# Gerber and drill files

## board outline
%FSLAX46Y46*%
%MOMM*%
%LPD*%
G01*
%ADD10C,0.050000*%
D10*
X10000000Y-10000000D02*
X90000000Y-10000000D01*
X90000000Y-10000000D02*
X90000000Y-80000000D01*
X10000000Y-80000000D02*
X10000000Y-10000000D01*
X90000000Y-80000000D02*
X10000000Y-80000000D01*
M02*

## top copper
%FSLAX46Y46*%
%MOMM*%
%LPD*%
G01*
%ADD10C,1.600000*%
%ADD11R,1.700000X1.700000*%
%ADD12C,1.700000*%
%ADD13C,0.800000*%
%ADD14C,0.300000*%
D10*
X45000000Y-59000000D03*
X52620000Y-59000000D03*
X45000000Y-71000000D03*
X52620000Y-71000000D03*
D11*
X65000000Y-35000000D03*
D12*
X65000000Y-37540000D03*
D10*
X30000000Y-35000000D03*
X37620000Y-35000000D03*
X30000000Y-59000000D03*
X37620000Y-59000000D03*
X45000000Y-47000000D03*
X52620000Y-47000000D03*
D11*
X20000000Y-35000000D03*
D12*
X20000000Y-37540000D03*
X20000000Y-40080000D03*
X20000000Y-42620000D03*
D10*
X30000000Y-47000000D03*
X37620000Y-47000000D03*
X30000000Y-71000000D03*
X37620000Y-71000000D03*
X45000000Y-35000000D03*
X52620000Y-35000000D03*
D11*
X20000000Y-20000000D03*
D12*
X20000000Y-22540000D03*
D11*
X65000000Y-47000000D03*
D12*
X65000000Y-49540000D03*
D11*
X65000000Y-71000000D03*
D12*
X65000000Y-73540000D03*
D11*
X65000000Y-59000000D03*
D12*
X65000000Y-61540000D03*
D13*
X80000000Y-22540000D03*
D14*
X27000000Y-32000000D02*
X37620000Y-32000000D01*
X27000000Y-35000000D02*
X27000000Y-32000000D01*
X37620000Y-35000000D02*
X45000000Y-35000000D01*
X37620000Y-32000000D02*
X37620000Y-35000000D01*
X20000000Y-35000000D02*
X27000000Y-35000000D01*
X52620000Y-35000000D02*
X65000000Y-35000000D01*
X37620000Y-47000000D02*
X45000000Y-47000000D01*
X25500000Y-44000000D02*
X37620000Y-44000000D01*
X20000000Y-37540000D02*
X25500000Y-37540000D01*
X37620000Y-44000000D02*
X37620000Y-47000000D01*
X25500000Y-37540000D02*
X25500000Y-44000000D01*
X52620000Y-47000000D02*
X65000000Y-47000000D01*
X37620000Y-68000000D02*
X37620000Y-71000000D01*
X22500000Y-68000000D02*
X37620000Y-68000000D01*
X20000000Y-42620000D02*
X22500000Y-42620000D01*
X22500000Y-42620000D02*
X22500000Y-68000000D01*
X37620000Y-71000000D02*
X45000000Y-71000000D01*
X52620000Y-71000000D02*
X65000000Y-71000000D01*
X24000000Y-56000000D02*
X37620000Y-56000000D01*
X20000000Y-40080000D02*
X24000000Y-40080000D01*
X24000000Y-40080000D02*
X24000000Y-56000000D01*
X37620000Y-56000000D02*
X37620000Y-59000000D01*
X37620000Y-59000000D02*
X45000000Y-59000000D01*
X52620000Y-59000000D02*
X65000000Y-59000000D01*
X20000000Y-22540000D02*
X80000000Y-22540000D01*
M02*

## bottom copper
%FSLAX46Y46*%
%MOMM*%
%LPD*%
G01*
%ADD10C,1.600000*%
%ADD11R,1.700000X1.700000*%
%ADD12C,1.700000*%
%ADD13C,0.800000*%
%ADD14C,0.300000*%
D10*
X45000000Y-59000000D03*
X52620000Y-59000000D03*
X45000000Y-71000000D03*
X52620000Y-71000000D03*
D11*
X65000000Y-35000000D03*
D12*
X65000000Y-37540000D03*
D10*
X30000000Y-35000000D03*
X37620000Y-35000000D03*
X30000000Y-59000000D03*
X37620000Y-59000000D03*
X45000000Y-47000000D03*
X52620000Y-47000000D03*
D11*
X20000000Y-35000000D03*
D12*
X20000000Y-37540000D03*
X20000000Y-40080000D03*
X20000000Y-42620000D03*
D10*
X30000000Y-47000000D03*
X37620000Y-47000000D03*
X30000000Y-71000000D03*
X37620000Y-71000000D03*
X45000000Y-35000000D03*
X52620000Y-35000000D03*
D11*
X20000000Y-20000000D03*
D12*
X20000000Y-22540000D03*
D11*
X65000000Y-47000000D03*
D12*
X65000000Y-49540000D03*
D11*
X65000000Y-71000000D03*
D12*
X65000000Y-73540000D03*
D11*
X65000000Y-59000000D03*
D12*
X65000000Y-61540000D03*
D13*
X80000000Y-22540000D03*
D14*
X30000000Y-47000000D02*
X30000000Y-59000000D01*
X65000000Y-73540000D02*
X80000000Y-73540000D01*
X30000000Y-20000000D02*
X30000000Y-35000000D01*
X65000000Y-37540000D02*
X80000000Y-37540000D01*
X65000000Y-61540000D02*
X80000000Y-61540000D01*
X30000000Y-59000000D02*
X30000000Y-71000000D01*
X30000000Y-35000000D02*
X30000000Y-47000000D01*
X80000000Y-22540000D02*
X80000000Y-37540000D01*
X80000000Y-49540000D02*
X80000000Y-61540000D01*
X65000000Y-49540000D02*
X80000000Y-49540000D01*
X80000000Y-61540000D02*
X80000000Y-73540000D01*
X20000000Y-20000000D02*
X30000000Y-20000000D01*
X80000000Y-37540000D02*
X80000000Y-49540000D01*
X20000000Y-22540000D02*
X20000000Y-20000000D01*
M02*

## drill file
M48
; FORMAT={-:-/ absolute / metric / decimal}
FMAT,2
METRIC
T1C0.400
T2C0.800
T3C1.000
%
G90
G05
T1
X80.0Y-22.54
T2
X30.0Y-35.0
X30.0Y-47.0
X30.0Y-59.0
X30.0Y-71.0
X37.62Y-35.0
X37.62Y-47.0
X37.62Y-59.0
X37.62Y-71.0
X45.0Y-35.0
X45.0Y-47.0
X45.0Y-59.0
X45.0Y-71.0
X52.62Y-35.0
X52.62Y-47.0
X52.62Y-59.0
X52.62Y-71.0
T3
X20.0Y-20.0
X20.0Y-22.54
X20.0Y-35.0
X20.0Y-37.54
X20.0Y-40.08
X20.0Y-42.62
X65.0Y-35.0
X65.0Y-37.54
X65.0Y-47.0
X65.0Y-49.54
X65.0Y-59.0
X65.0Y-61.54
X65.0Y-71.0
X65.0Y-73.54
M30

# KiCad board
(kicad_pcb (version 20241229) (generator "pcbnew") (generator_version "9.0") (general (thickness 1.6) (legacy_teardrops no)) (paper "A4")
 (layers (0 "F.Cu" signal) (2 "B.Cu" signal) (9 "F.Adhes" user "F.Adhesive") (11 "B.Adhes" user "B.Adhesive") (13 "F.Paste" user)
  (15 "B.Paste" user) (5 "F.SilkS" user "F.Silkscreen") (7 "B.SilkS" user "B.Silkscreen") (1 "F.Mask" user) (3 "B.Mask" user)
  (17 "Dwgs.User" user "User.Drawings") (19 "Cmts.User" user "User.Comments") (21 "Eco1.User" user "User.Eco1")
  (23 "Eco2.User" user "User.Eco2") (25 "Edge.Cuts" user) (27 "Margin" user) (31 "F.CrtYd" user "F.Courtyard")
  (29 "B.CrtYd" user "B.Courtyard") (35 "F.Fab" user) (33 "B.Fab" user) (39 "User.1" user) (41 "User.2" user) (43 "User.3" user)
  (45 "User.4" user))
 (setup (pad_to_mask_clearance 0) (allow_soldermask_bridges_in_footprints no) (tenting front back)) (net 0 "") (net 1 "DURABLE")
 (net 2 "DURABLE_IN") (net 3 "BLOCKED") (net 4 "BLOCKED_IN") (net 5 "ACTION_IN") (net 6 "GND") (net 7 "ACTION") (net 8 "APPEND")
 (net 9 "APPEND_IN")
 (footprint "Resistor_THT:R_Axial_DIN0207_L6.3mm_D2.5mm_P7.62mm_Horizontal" (layer "F.Cu") (at 45 59)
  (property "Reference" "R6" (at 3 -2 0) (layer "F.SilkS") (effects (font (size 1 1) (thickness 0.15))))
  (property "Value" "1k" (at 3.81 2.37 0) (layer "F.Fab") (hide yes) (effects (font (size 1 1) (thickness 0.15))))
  (pad "1" thru_hole circle (at 0 0) (size 1.6 1.6) (drill 0.8) (layers "*.Cu" "*.Mask") (remove_unused_layers no) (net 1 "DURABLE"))
  (pad "2" thru_hole circle (at 7.62 0) (size 1.6 1.6) (drill 0.8) (layers "*.Cu" "*.Mask") (remove_unused_layers no) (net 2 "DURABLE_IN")))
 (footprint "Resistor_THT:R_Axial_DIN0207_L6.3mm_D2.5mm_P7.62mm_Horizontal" (layer "F.Cu") (at 45 71)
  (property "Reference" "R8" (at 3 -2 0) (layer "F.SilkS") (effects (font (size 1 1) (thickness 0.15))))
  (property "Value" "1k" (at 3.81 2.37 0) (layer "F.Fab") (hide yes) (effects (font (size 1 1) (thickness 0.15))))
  (pad "1" thru_hole circle (at 0 0) (size 1.6 1.6) (drill 0.8) (layers "*.Cu" "*.Mask") (remove_unused_layers no) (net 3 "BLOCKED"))
  (pad "2" thru_hole circle (at 7.62 0) (size 1.6 1.6) (drill 0.8) (layers "*.Cu" "*.Mask") (remove_unused_layers no) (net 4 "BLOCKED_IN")))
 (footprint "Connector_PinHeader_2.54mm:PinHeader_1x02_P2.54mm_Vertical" (layer "F.Cu") (at 65 35)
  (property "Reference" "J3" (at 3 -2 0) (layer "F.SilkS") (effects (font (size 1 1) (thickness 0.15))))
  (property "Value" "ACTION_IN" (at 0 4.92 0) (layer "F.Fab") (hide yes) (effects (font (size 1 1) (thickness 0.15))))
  (pad "1" thru_hole rect (at 0 0) (size 1.7 1.7) (drill 1) (layers "*.Cu" "*.Mask") (remove_unused_layers no) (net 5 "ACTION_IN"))
  (pad "2" thru_hole circle (at 0 2.54) (size 1.7 1.7) (drill 1) (layers "*.Cu" "*.Mask") (remove_unused_layers no) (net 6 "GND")))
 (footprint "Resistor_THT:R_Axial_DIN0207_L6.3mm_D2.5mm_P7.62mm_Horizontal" (layer "F.Cu") (at 30 35)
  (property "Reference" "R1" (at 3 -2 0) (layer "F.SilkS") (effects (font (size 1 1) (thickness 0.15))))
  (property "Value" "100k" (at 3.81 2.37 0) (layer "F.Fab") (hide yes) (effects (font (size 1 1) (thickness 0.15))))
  (pad "1" thru_hole circle (at 0 0) (size 1.6 1.6) (drill 0.8) (layers "*.Cu" "*.Mask") (remove_unused_layers no) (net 6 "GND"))
  (pad "2" thru_hole circle (at 7.62 0) (size 1.6 1.6) (drill 0.8) (layers "*.Cu" "*.Mask") (remove_unused_layers no) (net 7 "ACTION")))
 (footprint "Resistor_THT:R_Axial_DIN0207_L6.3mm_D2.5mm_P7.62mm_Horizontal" (layer "F.Cu") (at 30 59)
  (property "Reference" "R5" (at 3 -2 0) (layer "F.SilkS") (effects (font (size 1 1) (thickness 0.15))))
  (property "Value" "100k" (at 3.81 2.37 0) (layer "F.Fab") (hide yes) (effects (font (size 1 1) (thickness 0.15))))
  (pad "1" thru_hole circle (at 0 0) (size 1.6 1.6) (drill 0.8) (layers "*.Cu" "*.Mask") (remove_unused_layers no) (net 6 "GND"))
  (pad "2" thru_hole circle (at 7.62 0) (size 1.6 1.6) (drill 0.8) (layers "*.Cu" "*.Mask") (remove_unused_layers no) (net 1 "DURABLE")))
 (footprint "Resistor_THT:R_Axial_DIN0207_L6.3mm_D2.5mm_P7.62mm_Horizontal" (layer "F.Cu") (at 45 47)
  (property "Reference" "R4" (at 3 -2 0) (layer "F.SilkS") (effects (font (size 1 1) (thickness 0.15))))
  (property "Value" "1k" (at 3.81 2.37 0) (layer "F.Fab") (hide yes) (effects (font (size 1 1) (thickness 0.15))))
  (pad "1" thru_hole circle (at 0 0) (size 1.6 1.6) (drill 0.8) (layers "*.Cu" "*.Mask") (remove_unused_layers no) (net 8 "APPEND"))
  (pad "2" thru_hole circle (at 7.62 0) (size 1.6 1.6) (drill 0.8) (layers "*.Cu" "*.Mask") (remove_unused_layers no) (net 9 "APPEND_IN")))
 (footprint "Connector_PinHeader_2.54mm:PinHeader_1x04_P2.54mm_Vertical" (layer "F.Cu") (at 20 35)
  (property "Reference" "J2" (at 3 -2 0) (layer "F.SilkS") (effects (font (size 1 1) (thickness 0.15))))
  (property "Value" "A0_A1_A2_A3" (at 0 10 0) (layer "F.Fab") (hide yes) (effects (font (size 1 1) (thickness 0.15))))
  (pad "1" thru_hole rect (at 0 0) (size 1.7 1.7) (drill 1) (layers "*.Cu" "*.Mask") (remove_unused_layers no) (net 7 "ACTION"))
  (pad "2" thru_hole circle (at 0 2.54) (size 1.7 1.7) (drill 1) (layers "*.Cu" "*.Mask") (remove_unused_layers no) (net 8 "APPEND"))
  (pad "3" thru_hole circle (at 0 5.08) (size 1.7 1.7) (drill 1) (layers "*.Cu" "*.Mask") (remove_unused_layers no) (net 1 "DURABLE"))
  (pad "4" thru_hole circle (at 0 7.62) (size 1.7 1.7) (drill 1) (layers "*.Cu" "*.Mask") (remove_unused_layers no) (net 3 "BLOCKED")))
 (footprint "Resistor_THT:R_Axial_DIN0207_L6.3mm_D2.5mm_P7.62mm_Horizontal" (layer "F.Cu") (at 30 47)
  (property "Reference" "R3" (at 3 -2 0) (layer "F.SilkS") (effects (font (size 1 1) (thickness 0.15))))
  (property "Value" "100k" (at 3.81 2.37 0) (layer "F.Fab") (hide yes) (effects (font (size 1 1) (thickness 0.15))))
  (pad "1" thru_hole circle (at 0 0) (size 1.6 1.6) (drill 0.8) (layers "*.Cu" "*.Mask") (remove_unused_layers no) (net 6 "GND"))
  (pad "2" thru_hole circle (at 7.62 0) (size 1.6 1.6) (drill 0.8) (layers "*.Cu" "*.Mask") (remove_unused_layers no) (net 8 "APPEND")))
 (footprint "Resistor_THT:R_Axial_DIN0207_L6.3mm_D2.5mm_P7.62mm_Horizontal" (layer "F.Cu") (at 30 71)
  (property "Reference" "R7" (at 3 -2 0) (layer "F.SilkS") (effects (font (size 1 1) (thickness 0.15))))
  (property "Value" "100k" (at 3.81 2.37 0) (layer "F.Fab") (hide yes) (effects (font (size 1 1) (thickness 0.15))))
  (pad "1" thru_hole circle (at 0 0) (size 1.6 1.6) (drill 0.8) (layers "*.Cu" "*.Mask") (remove_unused_layers no) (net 6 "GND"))
  (pad "2" thru_hole circle (at 7.62 0) (size 1.6 1.6) (drill 0.8) (layers "*.Cu" "*.Mask") (remove_unused_layers no) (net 3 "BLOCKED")))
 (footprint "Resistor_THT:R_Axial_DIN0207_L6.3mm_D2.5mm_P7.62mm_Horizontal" (layer "F.Cu") (at 45 35)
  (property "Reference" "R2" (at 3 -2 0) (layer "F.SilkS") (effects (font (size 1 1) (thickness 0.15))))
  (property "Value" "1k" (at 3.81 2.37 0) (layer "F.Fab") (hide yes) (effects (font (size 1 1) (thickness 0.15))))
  (pad "1" thru_hole circle (at 0 0) (size 1.6 1.6) (drill 0.8) (layers "*.Cu" "*.Mask") (remove_unused_layers no) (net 7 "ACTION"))
  (pad "2" thru_hole circle (at 7.62 0) (size 1.6 1.6) (drill 0.8) (layers "*.Cu" "*.Mask") (remove_unused_layers no) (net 5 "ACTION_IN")))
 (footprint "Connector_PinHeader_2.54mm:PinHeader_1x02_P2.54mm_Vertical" (layer "F.Cu") (at 20 20)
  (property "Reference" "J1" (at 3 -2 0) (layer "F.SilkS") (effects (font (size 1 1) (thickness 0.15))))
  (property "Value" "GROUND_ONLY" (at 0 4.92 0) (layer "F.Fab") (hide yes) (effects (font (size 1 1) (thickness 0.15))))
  (pad "1" thru_hole rect (at 0 0) (size 1.7 1.7) (drill 1) (layers "*.Cu" "*.Mask") (remove_unused_layers no) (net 6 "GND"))
  (pad "2" thru_hole circle (at 0 2.54) (size 1.7 1.7) (drill 1) (layers "*.Cu" "*.Mask") (remove_unused_layers no) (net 6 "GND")))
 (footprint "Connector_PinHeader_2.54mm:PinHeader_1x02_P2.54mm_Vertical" (layer "F.Cu") (at 65 47)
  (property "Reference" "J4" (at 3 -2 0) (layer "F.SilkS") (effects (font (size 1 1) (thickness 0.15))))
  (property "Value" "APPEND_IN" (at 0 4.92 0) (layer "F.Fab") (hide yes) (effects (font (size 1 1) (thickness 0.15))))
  (pad "1" thru_hole rect (at 0 0) (size 1.7 1.7) (drill 1) (layers "*.Cu" "*.Mask") (remove_unused_layers no) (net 9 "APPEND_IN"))
  (pad "2" thru_hole circle (at 0 2.54) (size 1.7 1.7) (drill 1) (layers "*.Cu" "*.Mask") (remove_unused_layers no) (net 6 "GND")))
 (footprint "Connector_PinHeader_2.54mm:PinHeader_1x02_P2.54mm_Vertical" (layer "F.Cu") (at 65 71)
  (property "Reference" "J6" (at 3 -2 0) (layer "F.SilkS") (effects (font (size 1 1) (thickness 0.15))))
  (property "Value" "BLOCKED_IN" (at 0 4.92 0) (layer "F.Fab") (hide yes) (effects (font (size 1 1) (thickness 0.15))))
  (pad "1" thru_hole rect (at 0 0) (size 1.7 1.7) (drill 1) (layers "*.Cu" "*.Mask") (remove_unused_layers no) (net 4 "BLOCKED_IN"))
  (pad "2" thru_hole circle (at 0 2.54) (size 1.7 1.7) (drill 1) (layers "*.Cu" "*.Mask") (remove_unused_layers no) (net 6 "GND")))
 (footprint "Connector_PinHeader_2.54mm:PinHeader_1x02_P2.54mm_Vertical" (layer "F.Cu") (at 65 59)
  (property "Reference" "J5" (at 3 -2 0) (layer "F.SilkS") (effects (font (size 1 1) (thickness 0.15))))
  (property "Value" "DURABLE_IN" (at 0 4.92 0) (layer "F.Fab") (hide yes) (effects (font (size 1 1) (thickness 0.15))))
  (pad "1" thru_hole rect (at 0 0) (size 1.7 1.7) (drill 1) (layers "*.Cu" "*.Mask") (remove_unused_layers no) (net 2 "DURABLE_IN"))
  (pad "2" thru_hole circle (at 0 2.54) (size 1.7 1.7) (drill 1) (layers "*.Cu" "*.Mask") (remove_unused_layers no) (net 6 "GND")))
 (gr_line (start 10 10) (end 90 10) (stroke (width 0.05) (type default)) (layer "Edge.Cuts"))
 (gr_line (start 90 10) (end 90 80) (stroke (width 0.05) (type default)) (layer "Edge.Cuts"))
 (gr_line (start 10 80) (end 10 10) (stroke (width 0.05) (type default)) (layer "Edge.Cuts"))
 (gr_line (start 90 80) (end 10 80) (stroke (width 0.05) (type default)) (layer "Edge.Cuts"))
 (segment (start 27 32) (end 37.62 32) (width 0.3) (layer "F.Cu") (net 7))
 (segment (start 27 35) (end 27 32) (width 0.3) (layer "F.Cu") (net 7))
 (segment (start 37.62 35) (end 45 35) (width 0.3) (layer "F.Cu") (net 7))
 (segment (start 37.62 32) (end 37.62 35) (width 0.3) (layer "F.Cu") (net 7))
 (segment (start 20 35) (end 27 35) (width 0.3) (layer "F.Cu") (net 7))
 (segment (start 52.62 35) (end 65 35) (width 0.3) (layer "F.Cu") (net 5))
 (segment (start 37.62 47) (end 45 47) (width 0.3) (layer "F.Cu") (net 8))
 (segment (start 25.5 44) (end 37.62 44) (width 0.3) (layer "F.Cu") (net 8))
 (segment (start 20 37.54) (end 25.5 37.54) (width 0.3) (layer "F.Cu") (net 8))
 (segment (start 37.62 44) (end 37.62 47) (width 0.3) (layer "F.Cu") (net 8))
 (segment (start 25.5 37.54) (end 25.5 44) (width 0.3) (layer "F.Cu") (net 8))
 (segment (start 52.62 47) (end 65 47) (width 0.3) (layer "F.Cu") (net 9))
 (segment (start 37.62 68) (end 37.62 71) (width 0.3) (layer "F.Cu") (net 3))
 (segment (start 22.5 68) (end 37.62 68) (width 0.3) (layer "F.Cu") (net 3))
 (segment (start 20 42.62) (end 22.5 42.62) (width 0.3) (layer "F.Cu") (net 3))
 (segment (start 22.5 42.62) (end 22.5 68) (width 0.3) (layer "F.Cu") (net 3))
 (segment (start 37.62 71) (end 45 71) (width 0.3) (layer "F.Cu") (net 3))
 (segment (start 52.62 71) (end 65 71) (width 0.3) (layer "F.Cu") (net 4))
 (segment (start 24 56) (end 37.62 56) (width 0.3) (layer "F.Cu") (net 1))
 (segment (start 20 40.08) (end 24 40.08) (width 0.3) (layer "F.Cu") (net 1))
 (segment (start 24 40.08) (end 24 56) (width 0.3) (layer "F.Cu") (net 1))
 (segment (start 37.62 56) (end 37.62 59) (width 0.3) (layer "F.Cu") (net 1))
 (segment (start 37.62 59) (end 45 59) (width 0.3) (layer "F.Cu") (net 1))
 (segment (start 52.62 59) (end 65 59) (width 0.3) (layer "F.Cu") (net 2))
 (segment (start 20 22.54) (end 80 22.54) (width 0.3) (layer "F.Cu") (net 6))
 (via (at 80 22.54) (size 0.8) (drill 0.4) (layers "F.Cu" "B.Cu") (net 6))
 (segment (start 30 47) (end 30 59) (width 0.3) (layer "B.Cu") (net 6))
 (segment (start 65 73.54) (end 80 73.54) (width 0.3) (layer "B.Cu") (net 6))
 (segment (start 30 20) (end 30 35) (width 0.3) (layer "B.Cu") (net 6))
 (segment (start 65 37.54) (end 80 37.54) (width 0.3) (layer "B.Cu") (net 6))
 (segment (start 65 61.54) (end 80 61.54) (width 0.3) (layer "B.Cu") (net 6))
 (segment (start 30 59) (end 30 71) (width 0.3) (layer "B.Cu") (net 6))
 (segment (start 30 35) (end 30 47) (width 0.3) (layer "B.Cu") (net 6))
 (segment (start 80 22.54) (end 80 37.54) (width 0.3) (layer "B.Cu") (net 6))
 (segment (start 80 49.54) (end 80 61.54) (width 0.3) (layer "B.Cu") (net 6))
 (segment (start 65 49.54) (end 80 49.54) (width 0.3) (layer "B.Cu") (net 6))
 (segment (start 80 61.54) (end 80 73.54) (width 0.3) (layer "B.Cu") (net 6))
 (segment (start 20 20) (end 30 20) (width 0.3) (layer "B.Cu") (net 6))
 (segment (start 80 37.54) (end 80 49.54) (width 0.3) (layer "B.Cu") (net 6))
 (segment (start 20 22.54) (end 20 20) (width 0.3) (layer "B.Cu") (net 6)))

